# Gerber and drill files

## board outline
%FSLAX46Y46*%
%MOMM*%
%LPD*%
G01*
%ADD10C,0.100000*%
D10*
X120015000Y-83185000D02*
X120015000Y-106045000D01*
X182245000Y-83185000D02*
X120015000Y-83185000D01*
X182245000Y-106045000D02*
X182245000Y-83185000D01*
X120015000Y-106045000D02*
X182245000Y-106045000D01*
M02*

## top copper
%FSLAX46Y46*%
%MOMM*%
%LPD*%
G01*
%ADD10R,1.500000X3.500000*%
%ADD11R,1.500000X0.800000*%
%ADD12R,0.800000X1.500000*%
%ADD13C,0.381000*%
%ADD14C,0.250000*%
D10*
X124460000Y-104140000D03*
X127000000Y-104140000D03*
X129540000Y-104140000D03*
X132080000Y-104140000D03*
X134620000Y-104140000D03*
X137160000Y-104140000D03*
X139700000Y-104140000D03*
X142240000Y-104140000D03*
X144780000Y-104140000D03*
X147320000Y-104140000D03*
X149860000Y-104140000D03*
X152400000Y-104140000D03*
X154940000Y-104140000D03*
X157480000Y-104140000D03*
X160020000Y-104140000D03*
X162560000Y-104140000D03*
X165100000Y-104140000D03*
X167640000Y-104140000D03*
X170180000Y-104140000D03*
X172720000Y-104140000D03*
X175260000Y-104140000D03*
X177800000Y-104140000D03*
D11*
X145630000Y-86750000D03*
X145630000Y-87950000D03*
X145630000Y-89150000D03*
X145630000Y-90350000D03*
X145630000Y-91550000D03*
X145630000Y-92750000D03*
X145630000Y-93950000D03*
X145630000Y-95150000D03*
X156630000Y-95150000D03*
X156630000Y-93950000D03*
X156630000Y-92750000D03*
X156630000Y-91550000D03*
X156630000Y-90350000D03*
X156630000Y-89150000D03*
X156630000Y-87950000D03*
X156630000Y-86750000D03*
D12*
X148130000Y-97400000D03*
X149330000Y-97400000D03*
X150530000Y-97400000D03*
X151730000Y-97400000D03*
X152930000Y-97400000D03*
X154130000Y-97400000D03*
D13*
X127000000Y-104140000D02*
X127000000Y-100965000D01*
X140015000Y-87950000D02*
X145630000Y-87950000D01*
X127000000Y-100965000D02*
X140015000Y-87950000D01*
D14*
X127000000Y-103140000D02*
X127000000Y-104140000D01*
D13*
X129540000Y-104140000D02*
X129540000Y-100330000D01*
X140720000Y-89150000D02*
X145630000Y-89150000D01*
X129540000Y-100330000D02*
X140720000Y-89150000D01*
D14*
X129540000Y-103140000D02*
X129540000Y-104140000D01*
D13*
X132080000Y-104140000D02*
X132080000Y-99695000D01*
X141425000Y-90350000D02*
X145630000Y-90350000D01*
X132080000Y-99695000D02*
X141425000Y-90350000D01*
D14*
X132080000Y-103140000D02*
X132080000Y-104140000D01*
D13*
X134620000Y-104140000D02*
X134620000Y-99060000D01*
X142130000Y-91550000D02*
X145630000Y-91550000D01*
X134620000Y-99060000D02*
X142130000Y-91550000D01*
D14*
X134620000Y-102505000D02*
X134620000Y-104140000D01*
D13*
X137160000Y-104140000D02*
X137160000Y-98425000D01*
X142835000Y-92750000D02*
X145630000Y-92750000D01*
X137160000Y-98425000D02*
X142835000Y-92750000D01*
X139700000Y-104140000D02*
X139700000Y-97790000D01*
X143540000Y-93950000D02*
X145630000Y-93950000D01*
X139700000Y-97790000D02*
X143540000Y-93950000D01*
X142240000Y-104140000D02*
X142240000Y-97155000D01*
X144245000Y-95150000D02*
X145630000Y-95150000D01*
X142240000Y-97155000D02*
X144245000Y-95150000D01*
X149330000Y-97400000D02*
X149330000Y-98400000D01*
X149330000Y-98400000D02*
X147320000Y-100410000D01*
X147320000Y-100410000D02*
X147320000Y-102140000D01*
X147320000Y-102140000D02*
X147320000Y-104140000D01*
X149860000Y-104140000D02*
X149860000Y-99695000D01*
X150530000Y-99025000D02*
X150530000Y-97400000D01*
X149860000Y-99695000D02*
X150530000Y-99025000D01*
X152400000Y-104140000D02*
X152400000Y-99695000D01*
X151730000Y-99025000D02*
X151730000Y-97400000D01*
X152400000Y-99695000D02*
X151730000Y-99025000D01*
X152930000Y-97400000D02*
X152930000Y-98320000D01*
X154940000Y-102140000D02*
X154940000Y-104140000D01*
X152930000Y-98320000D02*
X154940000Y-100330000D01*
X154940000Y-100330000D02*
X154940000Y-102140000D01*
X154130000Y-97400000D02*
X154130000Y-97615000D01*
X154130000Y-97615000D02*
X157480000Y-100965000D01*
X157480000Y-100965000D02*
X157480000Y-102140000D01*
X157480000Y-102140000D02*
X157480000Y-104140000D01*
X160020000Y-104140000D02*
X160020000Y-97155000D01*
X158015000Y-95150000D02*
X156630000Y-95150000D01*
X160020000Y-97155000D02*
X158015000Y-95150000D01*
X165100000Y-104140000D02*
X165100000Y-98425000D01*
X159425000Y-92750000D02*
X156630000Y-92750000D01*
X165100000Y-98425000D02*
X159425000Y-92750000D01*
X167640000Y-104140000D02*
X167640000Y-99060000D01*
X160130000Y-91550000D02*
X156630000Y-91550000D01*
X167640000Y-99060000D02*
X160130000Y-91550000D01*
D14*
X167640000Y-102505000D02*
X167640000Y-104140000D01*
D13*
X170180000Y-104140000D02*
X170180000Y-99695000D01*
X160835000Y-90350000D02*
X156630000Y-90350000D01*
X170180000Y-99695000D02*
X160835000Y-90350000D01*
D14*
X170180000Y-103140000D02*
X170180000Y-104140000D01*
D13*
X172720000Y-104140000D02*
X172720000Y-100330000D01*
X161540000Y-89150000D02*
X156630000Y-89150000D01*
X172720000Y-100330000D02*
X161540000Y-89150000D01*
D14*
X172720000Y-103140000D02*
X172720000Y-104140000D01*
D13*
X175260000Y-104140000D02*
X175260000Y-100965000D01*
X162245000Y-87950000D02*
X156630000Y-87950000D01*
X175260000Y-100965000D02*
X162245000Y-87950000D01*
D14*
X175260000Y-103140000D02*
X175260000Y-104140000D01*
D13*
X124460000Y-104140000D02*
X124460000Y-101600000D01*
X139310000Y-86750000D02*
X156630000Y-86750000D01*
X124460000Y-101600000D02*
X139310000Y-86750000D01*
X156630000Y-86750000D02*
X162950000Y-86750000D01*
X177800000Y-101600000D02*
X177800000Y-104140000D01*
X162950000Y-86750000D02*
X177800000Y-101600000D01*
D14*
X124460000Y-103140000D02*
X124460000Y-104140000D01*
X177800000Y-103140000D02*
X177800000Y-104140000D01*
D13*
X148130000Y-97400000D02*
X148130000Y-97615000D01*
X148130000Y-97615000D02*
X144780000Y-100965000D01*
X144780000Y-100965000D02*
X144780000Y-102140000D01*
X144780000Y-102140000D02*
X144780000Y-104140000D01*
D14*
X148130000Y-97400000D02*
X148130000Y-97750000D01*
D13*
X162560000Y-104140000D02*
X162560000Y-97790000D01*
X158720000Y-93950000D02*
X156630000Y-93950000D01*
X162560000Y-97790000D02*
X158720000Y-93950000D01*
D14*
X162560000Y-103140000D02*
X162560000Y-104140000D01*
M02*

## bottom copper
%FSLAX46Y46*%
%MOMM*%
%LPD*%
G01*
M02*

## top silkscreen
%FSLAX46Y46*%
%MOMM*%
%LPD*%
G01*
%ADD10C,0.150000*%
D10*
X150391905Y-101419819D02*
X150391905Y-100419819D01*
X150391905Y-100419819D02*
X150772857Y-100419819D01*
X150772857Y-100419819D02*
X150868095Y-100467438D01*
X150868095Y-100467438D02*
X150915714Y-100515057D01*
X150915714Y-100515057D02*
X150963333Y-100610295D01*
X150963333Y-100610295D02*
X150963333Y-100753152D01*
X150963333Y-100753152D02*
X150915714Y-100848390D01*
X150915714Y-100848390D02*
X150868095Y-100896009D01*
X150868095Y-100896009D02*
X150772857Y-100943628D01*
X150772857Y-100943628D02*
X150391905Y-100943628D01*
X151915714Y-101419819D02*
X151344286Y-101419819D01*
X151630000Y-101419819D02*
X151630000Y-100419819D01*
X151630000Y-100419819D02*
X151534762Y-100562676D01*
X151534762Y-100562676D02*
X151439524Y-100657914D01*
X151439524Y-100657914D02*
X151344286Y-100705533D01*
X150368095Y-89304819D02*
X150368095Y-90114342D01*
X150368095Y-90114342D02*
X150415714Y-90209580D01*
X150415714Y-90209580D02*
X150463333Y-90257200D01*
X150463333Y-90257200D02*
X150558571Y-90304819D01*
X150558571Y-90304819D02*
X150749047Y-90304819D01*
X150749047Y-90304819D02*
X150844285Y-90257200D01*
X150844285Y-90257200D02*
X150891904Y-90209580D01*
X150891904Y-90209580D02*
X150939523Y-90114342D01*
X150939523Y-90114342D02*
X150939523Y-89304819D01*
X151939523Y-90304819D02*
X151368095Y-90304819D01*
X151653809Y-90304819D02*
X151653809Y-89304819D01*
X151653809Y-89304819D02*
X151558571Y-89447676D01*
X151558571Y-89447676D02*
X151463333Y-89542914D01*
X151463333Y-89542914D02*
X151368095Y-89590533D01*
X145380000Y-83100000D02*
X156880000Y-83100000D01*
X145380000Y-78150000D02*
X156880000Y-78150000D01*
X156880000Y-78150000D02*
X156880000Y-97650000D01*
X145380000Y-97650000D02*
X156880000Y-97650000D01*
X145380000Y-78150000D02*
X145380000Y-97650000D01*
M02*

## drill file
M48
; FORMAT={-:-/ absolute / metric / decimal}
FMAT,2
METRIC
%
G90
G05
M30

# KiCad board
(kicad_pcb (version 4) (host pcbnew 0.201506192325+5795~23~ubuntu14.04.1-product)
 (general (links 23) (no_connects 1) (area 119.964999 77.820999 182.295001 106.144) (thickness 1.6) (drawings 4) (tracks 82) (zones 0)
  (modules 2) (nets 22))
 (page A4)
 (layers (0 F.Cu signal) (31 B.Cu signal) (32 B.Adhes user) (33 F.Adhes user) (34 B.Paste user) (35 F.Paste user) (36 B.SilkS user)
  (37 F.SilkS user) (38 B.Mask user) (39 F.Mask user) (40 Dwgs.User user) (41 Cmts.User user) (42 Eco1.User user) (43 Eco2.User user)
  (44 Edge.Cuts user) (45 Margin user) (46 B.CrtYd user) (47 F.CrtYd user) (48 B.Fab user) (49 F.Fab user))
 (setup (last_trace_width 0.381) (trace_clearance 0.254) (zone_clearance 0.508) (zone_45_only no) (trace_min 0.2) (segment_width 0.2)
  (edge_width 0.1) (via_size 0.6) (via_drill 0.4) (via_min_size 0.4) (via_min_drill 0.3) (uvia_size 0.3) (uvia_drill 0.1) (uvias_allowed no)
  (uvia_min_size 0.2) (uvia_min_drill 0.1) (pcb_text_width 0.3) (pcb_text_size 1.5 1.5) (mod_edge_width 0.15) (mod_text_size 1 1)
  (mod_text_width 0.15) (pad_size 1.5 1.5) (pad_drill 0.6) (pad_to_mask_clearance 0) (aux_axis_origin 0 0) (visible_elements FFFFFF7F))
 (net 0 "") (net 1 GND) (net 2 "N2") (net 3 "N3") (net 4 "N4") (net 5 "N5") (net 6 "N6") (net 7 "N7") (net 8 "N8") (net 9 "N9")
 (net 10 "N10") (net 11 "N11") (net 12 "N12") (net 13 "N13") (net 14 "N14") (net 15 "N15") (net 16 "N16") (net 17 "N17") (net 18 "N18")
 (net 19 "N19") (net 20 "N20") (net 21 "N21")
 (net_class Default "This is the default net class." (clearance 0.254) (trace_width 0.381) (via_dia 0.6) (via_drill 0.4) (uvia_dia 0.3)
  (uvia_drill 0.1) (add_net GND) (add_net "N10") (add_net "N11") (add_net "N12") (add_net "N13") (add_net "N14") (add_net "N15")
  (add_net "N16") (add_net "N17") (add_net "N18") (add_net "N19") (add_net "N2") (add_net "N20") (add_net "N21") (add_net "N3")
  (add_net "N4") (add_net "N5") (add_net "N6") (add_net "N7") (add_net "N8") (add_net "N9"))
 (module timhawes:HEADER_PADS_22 (layer F.Cu) (at 151.13 104.14)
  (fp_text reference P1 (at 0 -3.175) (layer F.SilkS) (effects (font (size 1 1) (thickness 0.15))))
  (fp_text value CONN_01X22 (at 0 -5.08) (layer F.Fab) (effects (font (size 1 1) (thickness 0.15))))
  (pad 1 smd rect (at -26.67 0) (size 1.5 3.5) (layers F.Cu F.Paste F.Mask) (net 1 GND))
  (pad 2 smd rect (at -24.13 0) (size 1.5 3.5) (layers F.Cu F.Paste F.Mask) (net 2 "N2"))
  (pad 3 smd rect (at -21.59 0) (size 1.5 3.5) (layers F.Cu F.Paste F.Mask) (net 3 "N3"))
  (pad 4 smd rect (at -19.05 0) (size 1.5 3.5) (layers F.Cu F.Paste F.Mask) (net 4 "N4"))
  (pad 5 smd rect (at -16.51 0) (size 1.5 3.5) (layers F.Cu F.Paste F.Mask) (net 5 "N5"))
  (pad 6 smd rect (at -13.97 0) (size 1.5 3.5) (layers F.Cu F.Paste F.Mask) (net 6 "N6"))
  (pad 7 smd rect (at -11.43 0) (size 1.5 3.5) (layers F.Cu F.Paste F.Mask) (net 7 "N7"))
  (pad 8 smd rect (at -8.89 0) (size 1.5 3.5) (layers F.Cu F.Paste F.Mask) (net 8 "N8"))
  (pad 9 smd rect (at -6.35 0) (size 1.5 3.5) (layers F.Cu F.Paste F.Mask) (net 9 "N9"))
  (pad 10 smd rect (at -3.81 0) (size 1.5 3.5) (layers F.Cu F.Paste F.Mask) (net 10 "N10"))
  (pad 11 smd rect (at -1.27 0) (size 1.5 3.5) (layers F.Cu F.Paste F.Mask) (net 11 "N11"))
  (pad 12 smd rect (at 1.27 0) (size 1.5 3.5) (layers F.Cu F.Paste F.Mask) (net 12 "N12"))
  (pad 13 smd rect (at 3.81 0) (size 1.5 3.5) (layers F.Cu F.Paste F.Mask) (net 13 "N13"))
  (pad 14 smd rect (at 6.35 0) (size 1.5 3.5) (layers F.Cu F.Paste F.Mask) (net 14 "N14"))
  (pad 15 smd rect (at 8.89 0) (size 1.5 3.5) (layers F.Cu F.Paste F.Mask) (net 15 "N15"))
  (pad 16 smd rect (at 11.43 0) (size 1.5 3.5) (layers F.Cu F.Paste F.Mask) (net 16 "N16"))
  (pad 17 smd rect (at 13.97 0) (size 1.5 3.5) (layers F.Cu F.Paste F.Mask) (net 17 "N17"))
  (pad 18 smd rect (at 16.51 0) (size 1.5 3.5) (layers F.Cu F.Paste F.Mask) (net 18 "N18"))
  (pad 19 smd rect (at 19.05 0) (size 1.5 3.5) (layers F.Cu F.Paste F.Mask) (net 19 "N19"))
  (pad 20 smd rect (at 21.59 0) (size 1.5 3.5) (layers F.Cu F.Paste F.Mask) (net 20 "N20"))
  (pad 21 smd rect (at 24.13 0) (size 1.5 3.5) (layers F.Cu F.Paste F.Mask) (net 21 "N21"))
  (pad 22 smd rect (at 26.67 0) (size 1.5 3.5) (layers F.Cu F.Paste F.Mask) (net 1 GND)))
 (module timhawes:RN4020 (layer F.Cu) (at 151.13 88.9)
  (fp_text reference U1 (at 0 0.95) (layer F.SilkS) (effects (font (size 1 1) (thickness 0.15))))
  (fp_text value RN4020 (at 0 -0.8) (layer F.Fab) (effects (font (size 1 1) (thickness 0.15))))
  (fp_line (start -5.75 -5.8) (end 5.75 -5.8) (layer F.SilkS) (width 0.15))
  (fp_line (start -5.75 -10.75) (end 5.75 -10.75) (layer F.SilkS) (width 0.15))
  (fp_line (start 5.75 -10.75) (end 5.75 8.75) (layer F.SilkS) (width 0.15))
  (fp_line (start -5.75 8.75) (end 5.75 8.75) (layer F.SilkS) (width 0.15))
  (fp_line (start -5.75 -10.75) (end -5.75 8.75) (layer F.SilkS) (width 0.15))
  (pad 1 smd rect (at -5.5 -2.15) (size 1.5 0.8) (layers F.Cu F.Paste F.Mask) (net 1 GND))
  (pad 2 smd rect (at -5.5 -0.95) (size 1.5 0.8) (layers F.Cu F.Paste F.Mask) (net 2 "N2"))
  (pad 3 smd rect (at -5.5 0.25) (size 1.5 0.8) (layers F.Cu F.Paste F.Mask) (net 3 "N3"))
  (pad 4 smd rect (at -5.5 1.45) (size 1.5 0.8) (layers F.Cu F.Paste F.Mask) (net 4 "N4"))
  (pad 5 smd rect (at -5.5 2.65) (size 1.5 0.8) (layers F.Cu F.Paste F.Mask) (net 5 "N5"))
  (pad 6 smd rect (at -5.5 3.85) (size 1.5 0.8) (layers F.Cu F.Paste F.Mask) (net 6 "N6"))
  (pad 7 smd rect (at -5.5 5.05) (size 1.5 0.8) (layers F.Cu F.Paste F.Mask) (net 7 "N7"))
  (pad 8 smd rect (at -5.5 6.25) (size 1.5 0.8) (layers F.Cu F.Paste F.Mask) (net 8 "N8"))
  (pad 17 smd rect (at 5.5 6.25) (size 1.5 0.8) (layers F.Cu F.Paste F.Mask) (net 15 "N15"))
  (pad 18 smd rect (at 5.5 5.05) (size 1.5 0.8) (layers F.Cu F.Paste F.Mask) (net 16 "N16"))
  (pad 19 smd rect (at 5.5 3.85) (size 1.5 0.8) (layers F.Cu F.Paste F.Mask) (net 17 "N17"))
  (pad 20 smd rect (at 5.5 2.65) (size 1.5 0.8) (layers F.Cu F.Paste F.Mask) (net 18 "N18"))
  (pad 21 smd rect (at 5.5 1.45) (size 1.5 0.8) (layers F.Cu F.Paste F.Mask) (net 19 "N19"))
  (pad 22 smd rect (at 5.5 0.25) (size 1.5 0.8) (layers F.Cu F.Paste F.Mask) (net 20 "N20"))
  (pad 23 smd rect (at 5.5 -0.95) (size 1.5 0.8) (layers F.Cu F.Paste F.Mask) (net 21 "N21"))
  (pad 24 smd rect (at 5.5 -2.15) (size 1.5 0.8) (layers F.Cu F.Paste F.Mask) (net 1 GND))
  (pad 10 smd rect (at -3 8.5 90) (size 1.5 0.8) (layers F.Cu F.Paste F.Mask) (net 9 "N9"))
  (pad 11 smd rect (at -1.8 8.5 90) (size 1.5 0.8) (layers F.Cu F.Paste F.Mask) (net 10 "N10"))
  (pad 12 smd rect (at -0.6 8.5 90) (size 1.5 0.8) (layers F.Cu F.Paste F.Mask) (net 11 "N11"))
  (pad 13 smd rect (at 0.6 8.5 90) (size 1.5 0.8) (layers F.Cu F.Paste F.Mask) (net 12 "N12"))
  (pad 14 smd rect (at 1.8 8.5 90) (size 1.5 0.8) (layers F.Cu F.Paste F.Mask) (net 13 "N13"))
  (pad 15 smd rect (at 3 8.5 90) (size 1.5 0.8) (layers F.Cu F.Paste F.Mask) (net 14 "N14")))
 (gr_line (start 120.015 83.185) (end 120.015 106.045) (angle 90) (layer Edge.Cuts) (width 0.1))
 (gr_line (start 182.245 83.185) (end 120.015 83.185) (angle 90) (layer Edge.Cuts) (width 0.1))
 (gr_line (start 182.245 106.045) (end 182.245 83.185) (angle 90) (layer Edge.Cuts) (width 0.1))
 (gr_line (start 120.015 106.045) (end 182.245 106.045) (angle 90) (layer Edge.Cuts) (width 0.1))
 (segment (start 127 104.14) (end 127 100.965) (width 0.381) (layer F.Cu) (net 2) (status 400000))
 (segment (start 140.015 87.95) (end 145.63 87.95) (width 0.381) (layer F.Cu) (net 2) (status 800000))
 (segment (start 127 100.965) (end 140.015 87.95) (width 0.381) (layer F.Cu) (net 2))
 (segment (start 127 103.14) (end 127 104.14) (width 0.25) (layer F.Cu) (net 2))
 (segment (start 129.54 104.14) (end 129.54 100.33) (width 0.381) (layer F.Cu) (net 3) (status 400000))
 (segment (start 140.72 89.15) (end 145.63 89.15) (width 0.381) (layer F.Cu) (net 3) (status 800000))
 (segment (start 129.54 100.33) (end 140.72 89.15) (width 0.381) (layer F.Cu) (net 3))
 (segment (start 129.54 103.14) (end 129.54 104.14) (width 0.25) (layer F.Cu) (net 3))
 (segment (start 132.08 104.14) (end 132.08 99.695) (width 0.381) (layer F.Cu) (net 4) (status 400000))
 (segment (start 141.425 90.35) (end 145.63 90.35) (width 0.381) (layer F.Cu) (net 4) (status 800000))
 (segment (start 132.08 99.695) (end 141.425 90.35) (width 0.381) (layer F.Cu) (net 4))
 (segment (start 132.08 103.14) (end 132.08 104.14) (width 0.25) (layer F.Cu) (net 4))
 (segment (start 134.62 104.14) (end 134.62 99.06) (width 0.381) (layer F.Cu) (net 5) (status 400000))
 (segment (start 142.13 91.55) (end 145.63 91.55) (width 0.381) (layer F.Cu) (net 5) (status 800000))
 (segment (start 134.62 99.06) (end 142.13 91.55) (width 0.381) (layer F.Cu) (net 5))
 (segment (start 134.62 102.505) (end 134.62 104.14) (width 0.25) (layer F.Cu) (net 5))
 (segment (start 137.16 104.14) (end 137.16 98.425) (width 0.381) (layer F.Cu) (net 6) (status 400000))
 (segment (start 142.835 92.75) (end 145.63 92.75) (width 0.381) (layer F.Cu) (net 6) (status 800000))
 (segment (start 137.16 98.425) (end 142.835 92.75) (width 0.381) (layer F.Cu) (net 6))
 (segment (start 139.7 104.14) (end 139.7 97.79) (width 0.381) (layer F.Cu) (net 7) (status 400000))
 (segment (start 143.54 93.95) (end 145.63 93.95) (width 0.381) (layer F.Cu) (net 7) (status 800000))
 (segment (start 139.7 97.79) (end 143.54 93.95) (width 0.381) (layer F.Cu) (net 7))
 (segment (start 142.24 104.14) (end 142.24 97.155) (width 0.381) (layer F.Cu) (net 8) (status 400000))
 (segment (start 144.245 95.15) (end 145.63 95.15) (width 0.381) (layer F.Cu) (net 8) (status 800000))
 (segment (start 142.24 97.155) (end 144.245 95.15) (width 0.381) (layer F.Cu) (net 8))
 (segment (start 149.33 97.4) (end 149.33 98.4) (width 0.381) (layer F.Cu) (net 10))
 (segment (start 149.33 98.4) (end 147.32 100.41) (width 0.381) (layer F.Cu) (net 10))
 (segment (start 147.32 100.41) (end 147.32 102.14) (width 0.381) (layer F.Cu) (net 10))
 (segment (start 147.32 102.14) (end 147.32 104.14) (width 0.381) (layer F.Cu) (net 10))
 (segment (start 149.86 104.14) (end 149.86 99.695) (width 0.381) (layer F.Cu) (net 11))
 (segment (start 150.53 99.025) (end 150.53 97.4) (width 0.381) (layer F.Cu) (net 11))
 (segment (start 149.86 99.695) (end 150.53 99.025) (width 0.381) (layer F.Cu) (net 11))
 (segment (start 152.4 104.14) (end 152.4 99.695) (width 0.381) (layer F.Cu) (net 12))
 (segment (start 151.73 99.025) (end 151.73 97.4) (width 0.381) (layer F.Cu) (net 12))
 (segment (start 152.4 99.695) (end 151.73 99.025) (width 0.381) (layer F.Cu) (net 12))
 (segment (start 152.93 97.4) (end 152.93 98.32) (width 0.381) (layer F.Cu) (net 13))
 (segment (start 154.94 102.14) (end 154.94 104.14) (width 0.381) (layer F.Cu) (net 13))
 (segment (start 152.93 98.32) (end 154.94 100.33) (width 0.381) (layer F.Cu) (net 13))
 (segment (start 154.94 100.33) (end 154.94 102.14) (width 0.381) (layer F.Cu) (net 13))
 (segment (start 154.13 97.4) (end 154.13 97.615) (width 0.381) (layer F.Cu) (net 14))
 (segment (start 154.13 97.615) (end 157.48 100.965) (width 0.381) (layer F.Cu) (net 14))
 (segment (start 157.48 100.965) (end 157.48 102.14) (width 0.381) (layer F.Cu) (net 14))
 (segment (start 157.48 102.14) (end 157.48 104.14) (width 0.381) (layer F.Cu) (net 14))
 (segment (start 160.02 104.14) (end 160.02 97.155) (width 0.381) (layer F.Cu) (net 15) (status 400000))
 (segment (start 158.015 95.15) (end 156.63 95.15) (width 0.381) (layer F.Cu) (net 15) (status 800000))
 (segment (start 160.02 97.155) (end 158.015 95.15) (width 0.381) (layer F.Cu) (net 15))
 (segment (start 165.1 104.14) (end 165.1 98.425) (width 0.381) (layer F.Cu) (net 17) (status 400000))
 (segment (start 159.425 92.75) (end 156.63 92.75) (width 0.381) (layer F.Cu) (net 17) (status 800000))
 (segment (start 165.1 98.425) (end 159.425 92.75) (width 0.381) (layer F.Cu) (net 17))
 (segment (start 167.64 104.14) (end 167.64 99.06) (width 0.381) (layer F.Cu) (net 18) (status 400000))
 (segment (start 160.13 91.55) (end 156.63 91.55) (width 0.381) (layer F.Cu) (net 18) (status 800000))
 (segment (start 167.64 99.06) (end 160.13 91.55) (width 0.381) (layer F.Cu) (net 18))
 (segment (start 167.64 102.505) (end 167.64 104.14) (width 0.25) (layer F.Cu) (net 18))
 (segment (start 170.18 104.14) (end 170.18 99.695) (width 0.381) (layer F.Cu) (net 19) (status 400000))
 (segment (start 160.835 90.35) (end 156.63 90.35) (width 0.381) (layer F.Cu) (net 19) (status 800000))
 (segment (start 170.18 99.695) (end 160.835 90.35) (width 0.381) (layer F.Cu) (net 19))
 (segment (start 170.18 103.14) (end 170.18 104.14) (width 0.25) (layer F.Cu) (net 19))
 (segment (start 172.72 104.14) (end 172.72 100.33) (width 0.381) (layer F.Cu) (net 20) (status 400000))
 (segment (start 161.54 89.15) (end 156.63 89.15) (width 0.381) (layer F.Cu) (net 20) (status 800000))
 (segment (start 172.72 100.33) (end 161.54 89.15) (width 0.381) (layer F.Cu) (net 20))
 (segment (start 172.72 103.14) (end 172.72 104.14) (width 0.25) (layer F.Cu) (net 20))
 (segment (start 175.26 104.14) (end 175.26 100.965) (width 0.381) (layer F.Cu) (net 21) (status 400000))
 (segment (start 162.245 87.95) (end 156.63 87.95) (width 0.381) (layer F.Cu) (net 21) (status 800000))
 (segment (start 175.26 100.965) (end 162.245 87.95) (width 0.381) (layer F.Cu) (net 21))
 (segment (start 175.26 103.14) (end 175.26 104.14) (width 0.25) (layer F.Cu) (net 21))
 (segment (start 124.46 104.14) (end 124.46 101.6) (width 0.381) (layer F.Cu) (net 1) (status 400000))
 (segment (start 139.31 86.75) (end 156.63 86.75) (width 0.381) (layer F.Cu) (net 1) (status 800000))
 (segment (start 124.46 101.6) (end 139.31 86.75) (width 0.381) (layer F.Cu) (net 1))
 (segment (start 156.63 86.75) (end 162.95 86.75) (width 0.381) (layer F.Cu) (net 1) (status 400000))
 (segment (start 177.8 101.6) (end 177.8 104.14) (width 0.381) (layer F.Cu) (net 1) (status 800000))
 (segment (start 162.95 86.75) (end 177.8 101.6) (width 0.381) (layer F.Cu) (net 1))
 (segment (start 124.46 103.14) (end 124.46 104.14) (width 0.25) (layer F.Cu) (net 1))
 (segment (start 177.8 103.14) (end 177.8 104.14) (width 0.25) (layer F.Cu) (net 1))
 (segment (start 148.13 97.4) (end 148.13 97.615) (width 0.381) (layer F.Cu) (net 9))
 (segment (start 148.13 97.615) (end 144.78 100.965) (width 0.381) (layer F.Cu) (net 9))
 (segment (start 144.78 100.965) (end 144.78 102.14) (width 0.381) (layer F.Cu) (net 9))
 (segment (start 144.78 102.14) (end 144.78 104.14) (width 0.381) (layer F.Cu) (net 9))
 (segment (start 148.13 97.4) (end 148.13 97.75) (width 0.25) (layer F.Cu) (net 9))
 (segment (start 162.56 104.14) (end 162.56 97.79) (width 0.381) (layer F.Cu) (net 16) (status 400000))
 (segment (start 158.72 93.95) (end 156.63 93.95) (width 0.381) (layer F.Cu) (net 16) (status 800000))
 (segment (start 162.56 97.79) (end 158.72 93.95) (width 0.381) (layer F.Cu) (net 16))
 (segment (start 162.56 103.14) (end 162.56 104.14) (width 0.25) (layer F.Cu) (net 16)))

